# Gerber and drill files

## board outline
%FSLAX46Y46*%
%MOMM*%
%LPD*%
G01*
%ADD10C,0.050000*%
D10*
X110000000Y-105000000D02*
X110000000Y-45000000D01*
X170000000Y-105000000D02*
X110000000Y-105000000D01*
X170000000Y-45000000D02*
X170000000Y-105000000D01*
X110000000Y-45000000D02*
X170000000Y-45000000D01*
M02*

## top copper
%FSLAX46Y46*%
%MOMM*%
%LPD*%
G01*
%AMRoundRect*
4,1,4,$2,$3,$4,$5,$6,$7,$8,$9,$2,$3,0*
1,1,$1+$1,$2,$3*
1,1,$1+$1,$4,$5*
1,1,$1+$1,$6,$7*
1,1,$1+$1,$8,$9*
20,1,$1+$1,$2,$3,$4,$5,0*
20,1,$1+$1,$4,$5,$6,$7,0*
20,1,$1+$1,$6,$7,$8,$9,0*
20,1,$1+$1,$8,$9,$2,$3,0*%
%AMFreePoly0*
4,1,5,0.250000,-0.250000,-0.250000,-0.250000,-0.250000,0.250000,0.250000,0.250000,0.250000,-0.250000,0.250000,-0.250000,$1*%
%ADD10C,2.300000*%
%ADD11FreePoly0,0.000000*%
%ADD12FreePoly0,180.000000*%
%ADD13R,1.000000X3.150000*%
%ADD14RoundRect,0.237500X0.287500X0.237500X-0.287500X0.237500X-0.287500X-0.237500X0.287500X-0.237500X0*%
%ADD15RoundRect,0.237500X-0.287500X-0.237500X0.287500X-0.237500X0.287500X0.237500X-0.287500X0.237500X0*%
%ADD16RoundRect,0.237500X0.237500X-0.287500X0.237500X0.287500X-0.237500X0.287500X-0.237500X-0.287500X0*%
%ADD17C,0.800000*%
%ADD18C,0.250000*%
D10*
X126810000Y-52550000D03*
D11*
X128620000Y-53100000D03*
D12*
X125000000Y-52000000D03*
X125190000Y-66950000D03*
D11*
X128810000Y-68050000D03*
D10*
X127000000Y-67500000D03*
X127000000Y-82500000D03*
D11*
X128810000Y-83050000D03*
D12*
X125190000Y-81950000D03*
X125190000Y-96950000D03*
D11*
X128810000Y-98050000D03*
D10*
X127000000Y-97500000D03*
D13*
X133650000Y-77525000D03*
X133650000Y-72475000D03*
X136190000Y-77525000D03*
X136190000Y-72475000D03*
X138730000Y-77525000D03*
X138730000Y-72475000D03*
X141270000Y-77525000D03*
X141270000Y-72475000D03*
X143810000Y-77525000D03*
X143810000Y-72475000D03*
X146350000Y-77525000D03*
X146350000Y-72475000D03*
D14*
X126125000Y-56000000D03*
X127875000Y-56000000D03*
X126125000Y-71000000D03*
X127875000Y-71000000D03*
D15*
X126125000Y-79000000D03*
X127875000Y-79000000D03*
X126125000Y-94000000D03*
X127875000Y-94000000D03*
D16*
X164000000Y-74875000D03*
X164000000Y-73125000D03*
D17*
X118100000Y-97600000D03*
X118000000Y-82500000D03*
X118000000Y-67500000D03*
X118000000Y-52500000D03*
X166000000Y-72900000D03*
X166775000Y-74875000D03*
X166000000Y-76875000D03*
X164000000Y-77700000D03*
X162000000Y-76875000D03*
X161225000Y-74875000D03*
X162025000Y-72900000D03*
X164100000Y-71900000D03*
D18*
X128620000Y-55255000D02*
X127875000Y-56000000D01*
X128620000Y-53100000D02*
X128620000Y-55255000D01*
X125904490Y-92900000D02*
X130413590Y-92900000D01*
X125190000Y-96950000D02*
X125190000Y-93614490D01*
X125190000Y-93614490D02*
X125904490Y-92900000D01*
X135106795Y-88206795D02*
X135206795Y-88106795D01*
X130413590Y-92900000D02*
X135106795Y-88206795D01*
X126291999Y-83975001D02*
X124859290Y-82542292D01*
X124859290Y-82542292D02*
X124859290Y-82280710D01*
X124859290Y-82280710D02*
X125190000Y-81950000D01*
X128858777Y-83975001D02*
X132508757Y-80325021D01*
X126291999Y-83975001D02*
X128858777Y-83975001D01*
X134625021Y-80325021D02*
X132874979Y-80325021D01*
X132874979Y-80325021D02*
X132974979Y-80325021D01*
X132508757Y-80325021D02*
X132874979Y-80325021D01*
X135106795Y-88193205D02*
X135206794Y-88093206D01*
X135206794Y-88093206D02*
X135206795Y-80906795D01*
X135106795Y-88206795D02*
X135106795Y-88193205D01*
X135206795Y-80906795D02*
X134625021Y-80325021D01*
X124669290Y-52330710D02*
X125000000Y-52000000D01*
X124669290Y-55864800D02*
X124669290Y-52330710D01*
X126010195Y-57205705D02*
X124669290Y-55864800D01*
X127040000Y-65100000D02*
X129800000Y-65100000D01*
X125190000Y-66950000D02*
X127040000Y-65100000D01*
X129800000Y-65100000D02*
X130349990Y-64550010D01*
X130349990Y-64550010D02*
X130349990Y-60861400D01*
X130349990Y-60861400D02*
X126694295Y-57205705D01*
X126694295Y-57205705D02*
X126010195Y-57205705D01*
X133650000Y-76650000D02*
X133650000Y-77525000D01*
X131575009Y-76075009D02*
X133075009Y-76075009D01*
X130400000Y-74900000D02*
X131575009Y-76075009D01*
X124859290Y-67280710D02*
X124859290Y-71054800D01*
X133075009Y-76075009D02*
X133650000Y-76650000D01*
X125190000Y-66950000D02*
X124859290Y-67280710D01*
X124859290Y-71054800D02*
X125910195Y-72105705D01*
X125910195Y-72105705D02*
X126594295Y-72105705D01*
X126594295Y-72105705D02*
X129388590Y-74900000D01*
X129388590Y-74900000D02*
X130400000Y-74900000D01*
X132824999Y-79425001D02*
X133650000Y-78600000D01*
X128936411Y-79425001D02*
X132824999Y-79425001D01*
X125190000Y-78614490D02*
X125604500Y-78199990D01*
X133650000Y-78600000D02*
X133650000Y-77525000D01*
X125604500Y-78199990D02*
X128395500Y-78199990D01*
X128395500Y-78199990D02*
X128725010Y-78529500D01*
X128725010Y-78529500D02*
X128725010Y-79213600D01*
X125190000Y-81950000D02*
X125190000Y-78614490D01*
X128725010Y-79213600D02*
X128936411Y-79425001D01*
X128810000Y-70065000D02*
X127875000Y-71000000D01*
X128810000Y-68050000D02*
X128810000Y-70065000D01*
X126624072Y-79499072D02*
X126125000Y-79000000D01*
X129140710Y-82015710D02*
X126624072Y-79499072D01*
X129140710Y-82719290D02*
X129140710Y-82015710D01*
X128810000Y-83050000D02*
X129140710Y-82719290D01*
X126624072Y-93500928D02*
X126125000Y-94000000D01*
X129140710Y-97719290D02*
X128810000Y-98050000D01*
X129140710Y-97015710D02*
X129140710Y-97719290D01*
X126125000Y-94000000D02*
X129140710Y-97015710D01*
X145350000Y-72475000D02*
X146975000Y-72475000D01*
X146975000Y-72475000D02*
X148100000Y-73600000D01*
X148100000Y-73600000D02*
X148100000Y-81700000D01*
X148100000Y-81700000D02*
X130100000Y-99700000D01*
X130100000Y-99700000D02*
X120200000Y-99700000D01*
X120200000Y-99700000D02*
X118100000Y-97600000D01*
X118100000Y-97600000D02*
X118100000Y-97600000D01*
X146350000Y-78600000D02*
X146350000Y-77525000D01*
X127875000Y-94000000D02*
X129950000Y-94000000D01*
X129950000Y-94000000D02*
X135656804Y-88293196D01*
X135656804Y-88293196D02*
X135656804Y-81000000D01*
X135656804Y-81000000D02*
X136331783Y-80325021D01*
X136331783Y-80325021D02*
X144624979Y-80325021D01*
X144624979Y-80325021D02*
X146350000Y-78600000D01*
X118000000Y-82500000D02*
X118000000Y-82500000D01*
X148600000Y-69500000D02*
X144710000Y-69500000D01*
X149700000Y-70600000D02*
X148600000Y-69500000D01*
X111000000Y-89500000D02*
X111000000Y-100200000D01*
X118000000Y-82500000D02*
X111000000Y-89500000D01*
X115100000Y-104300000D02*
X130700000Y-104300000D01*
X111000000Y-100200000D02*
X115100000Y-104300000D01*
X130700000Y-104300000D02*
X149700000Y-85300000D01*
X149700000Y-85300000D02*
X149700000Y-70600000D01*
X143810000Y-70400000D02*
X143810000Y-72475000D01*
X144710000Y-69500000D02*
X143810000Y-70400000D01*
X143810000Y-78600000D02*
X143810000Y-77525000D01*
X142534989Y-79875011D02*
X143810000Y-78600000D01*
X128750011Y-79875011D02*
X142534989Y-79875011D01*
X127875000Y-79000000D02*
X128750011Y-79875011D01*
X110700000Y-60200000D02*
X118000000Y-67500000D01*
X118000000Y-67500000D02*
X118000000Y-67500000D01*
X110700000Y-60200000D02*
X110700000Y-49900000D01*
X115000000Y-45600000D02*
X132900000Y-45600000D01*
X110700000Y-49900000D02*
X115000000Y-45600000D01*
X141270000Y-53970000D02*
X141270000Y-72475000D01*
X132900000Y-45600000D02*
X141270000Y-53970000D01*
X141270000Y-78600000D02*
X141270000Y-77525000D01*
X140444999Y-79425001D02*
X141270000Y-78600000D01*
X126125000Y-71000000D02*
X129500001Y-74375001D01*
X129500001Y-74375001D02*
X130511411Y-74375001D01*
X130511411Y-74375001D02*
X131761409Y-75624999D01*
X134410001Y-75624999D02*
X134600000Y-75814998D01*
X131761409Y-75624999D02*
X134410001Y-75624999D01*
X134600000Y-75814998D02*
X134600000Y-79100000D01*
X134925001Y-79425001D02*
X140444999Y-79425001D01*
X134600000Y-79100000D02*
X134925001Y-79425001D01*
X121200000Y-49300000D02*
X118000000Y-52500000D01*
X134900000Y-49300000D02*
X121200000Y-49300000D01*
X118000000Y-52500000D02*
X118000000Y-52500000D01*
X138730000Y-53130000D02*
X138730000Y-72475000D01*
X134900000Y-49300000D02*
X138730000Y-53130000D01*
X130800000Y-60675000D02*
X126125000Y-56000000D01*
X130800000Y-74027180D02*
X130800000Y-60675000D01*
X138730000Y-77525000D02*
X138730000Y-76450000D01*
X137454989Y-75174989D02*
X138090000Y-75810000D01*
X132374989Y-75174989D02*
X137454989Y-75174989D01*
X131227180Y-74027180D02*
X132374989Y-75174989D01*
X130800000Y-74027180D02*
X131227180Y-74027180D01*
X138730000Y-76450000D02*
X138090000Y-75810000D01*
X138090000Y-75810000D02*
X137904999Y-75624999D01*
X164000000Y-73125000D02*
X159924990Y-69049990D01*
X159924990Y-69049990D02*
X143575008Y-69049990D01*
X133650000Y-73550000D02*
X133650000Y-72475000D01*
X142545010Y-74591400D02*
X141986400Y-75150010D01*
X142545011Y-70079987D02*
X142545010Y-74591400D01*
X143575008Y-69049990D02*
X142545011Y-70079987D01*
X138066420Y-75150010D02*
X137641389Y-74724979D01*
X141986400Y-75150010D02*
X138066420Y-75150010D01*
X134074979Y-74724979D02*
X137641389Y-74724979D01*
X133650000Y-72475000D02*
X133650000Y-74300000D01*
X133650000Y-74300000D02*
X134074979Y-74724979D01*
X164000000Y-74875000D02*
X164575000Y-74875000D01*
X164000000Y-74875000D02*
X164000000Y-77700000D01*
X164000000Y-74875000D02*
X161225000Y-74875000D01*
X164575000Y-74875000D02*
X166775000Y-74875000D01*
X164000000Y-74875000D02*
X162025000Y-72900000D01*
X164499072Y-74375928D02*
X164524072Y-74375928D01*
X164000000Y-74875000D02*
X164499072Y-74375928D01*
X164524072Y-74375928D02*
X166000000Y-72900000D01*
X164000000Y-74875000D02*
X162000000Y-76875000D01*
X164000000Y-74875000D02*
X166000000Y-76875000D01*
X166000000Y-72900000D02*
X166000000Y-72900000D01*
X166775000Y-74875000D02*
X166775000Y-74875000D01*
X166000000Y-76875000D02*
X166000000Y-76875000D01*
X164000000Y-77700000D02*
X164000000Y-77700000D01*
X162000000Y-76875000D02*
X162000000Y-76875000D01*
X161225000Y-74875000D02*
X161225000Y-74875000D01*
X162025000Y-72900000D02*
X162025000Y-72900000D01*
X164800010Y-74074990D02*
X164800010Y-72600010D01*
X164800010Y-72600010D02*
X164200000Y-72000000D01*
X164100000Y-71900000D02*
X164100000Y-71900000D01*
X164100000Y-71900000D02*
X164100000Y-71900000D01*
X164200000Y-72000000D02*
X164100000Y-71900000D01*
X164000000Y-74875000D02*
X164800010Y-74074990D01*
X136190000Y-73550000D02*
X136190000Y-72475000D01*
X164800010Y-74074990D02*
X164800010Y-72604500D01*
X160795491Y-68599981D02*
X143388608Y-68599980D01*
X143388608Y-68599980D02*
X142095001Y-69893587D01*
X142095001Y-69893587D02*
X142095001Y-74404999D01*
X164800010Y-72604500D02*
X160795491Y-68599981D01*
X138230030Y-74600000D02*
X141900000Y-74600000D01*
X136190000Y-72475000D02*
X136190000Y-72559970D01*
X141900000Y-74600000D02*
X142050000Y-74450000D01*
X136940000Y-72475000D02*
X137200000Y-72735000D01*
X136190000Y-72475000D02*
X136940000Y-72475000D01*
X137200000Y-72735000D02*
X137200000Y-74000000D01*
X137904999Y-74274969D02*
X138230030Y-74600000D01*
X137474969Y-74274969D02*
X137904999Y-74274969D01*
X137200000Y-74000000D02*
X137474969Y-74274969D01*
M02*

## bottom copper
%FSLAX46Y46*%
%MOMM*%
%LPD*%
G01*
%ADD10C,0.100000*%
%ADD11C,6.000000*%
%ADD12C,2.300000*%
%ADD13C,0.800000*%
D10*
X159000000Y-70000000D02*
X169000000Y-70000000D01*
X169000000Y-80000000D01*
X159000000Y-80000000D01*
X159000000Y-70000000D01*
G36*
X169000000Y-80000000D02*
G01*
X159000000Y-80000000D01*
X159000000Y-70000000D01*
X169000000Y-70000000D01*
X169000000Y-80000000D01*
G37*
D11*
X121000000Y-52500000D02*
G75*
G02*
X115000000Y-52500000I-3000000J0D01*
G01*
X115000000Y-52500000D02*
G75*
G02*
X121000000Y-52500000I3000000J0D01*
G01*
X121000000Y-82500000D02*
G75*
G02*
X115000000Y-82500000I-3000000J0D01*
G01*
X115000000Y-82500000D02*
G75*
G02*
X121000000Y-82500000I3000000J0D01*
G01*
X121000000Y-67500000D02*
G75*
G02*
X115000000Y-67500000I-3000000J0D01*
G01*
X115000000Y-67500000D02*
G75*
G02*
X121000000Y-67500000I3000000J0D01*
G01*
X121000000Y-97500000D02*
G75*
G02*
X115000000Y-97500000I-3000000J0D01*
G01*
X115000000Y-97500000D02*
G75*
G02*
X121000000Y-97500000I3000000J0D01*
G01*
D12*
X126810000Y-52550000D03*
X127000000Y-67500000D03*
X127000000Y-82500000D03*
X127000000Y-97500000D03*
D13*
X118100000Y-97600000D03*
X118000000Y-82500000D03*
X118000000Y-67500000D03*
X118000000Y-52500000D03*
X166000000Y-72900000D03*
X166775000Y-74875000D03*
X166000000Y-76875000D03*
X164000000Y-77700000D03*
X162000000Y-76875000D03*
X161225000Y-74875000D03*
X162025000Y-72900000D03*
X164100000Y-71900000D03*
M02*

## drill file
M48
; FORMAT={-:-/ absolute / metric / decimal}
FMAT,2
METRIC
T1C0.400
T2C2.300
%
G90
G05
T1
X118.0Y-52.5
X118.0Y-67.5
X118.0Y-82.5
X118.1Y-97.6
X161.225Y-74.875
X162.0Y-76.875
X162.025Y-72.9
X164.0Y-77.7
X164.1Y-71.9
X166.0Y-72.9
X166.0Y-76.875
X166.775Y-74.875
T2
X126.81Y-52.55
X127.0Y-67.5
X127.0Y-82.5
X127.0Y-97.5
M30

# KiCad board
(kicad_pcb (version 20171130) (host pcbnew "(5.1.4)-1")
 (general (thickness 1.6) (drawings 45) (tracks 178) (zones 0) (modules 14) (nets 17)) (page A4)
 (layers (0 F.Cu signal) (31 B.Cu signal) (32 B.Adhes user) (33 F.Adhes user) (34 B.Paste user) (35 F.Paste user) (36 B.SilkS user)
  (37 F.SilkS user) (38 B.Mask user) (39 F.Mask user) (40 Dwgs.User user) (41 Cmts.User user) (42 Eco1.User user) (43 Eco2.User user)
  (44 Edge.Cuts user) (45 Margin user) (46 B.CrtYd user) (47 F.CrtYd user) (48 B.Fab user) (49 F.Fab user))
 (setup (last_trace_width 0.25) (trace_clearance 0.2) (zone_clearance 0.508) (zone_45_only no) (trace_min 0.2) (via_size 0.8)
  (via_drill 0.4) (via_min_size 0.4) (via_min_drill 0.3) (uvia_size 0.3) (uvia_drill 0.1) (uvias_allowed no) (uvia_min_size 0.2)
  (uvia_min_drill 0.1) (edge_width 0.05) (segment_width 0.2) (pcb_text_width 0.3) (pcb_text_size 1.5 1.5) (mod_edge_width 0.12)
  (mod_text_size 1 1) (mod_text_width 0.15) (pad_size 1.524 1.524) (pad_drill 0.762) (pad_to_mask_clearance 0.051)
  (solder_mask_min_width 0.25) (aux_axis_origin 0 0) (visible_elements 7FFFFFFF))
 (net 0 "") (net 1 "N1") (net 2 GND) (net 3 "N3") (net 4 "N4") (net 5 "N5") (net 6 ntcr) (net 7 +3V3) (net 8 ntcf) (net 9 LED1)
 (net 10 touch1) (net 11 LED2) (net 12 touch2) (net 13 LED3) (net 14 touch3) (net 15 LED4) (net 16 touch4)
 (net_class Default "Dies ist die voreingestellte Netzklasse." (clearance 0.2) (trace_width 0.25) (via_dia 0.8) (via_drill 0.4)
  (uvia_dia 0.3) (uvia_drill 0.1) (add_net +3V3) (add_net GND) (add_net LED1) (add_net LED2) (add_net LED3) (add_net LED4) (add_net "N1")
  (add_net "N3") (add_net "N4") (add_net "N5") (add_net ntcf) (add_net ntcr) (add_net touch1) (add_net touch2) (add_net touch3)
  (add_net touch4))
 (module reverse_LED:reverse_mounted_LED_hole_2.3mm (layer F.Cu) (at 126.81 52.55)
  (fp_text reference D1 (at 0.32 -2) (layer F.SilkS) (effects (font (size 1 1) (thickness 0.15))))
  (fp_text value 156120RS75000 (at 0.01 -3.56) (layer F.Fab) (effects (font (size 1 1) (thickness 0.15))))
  (pad 0 thru_hole circle (at 0 0) (size 2.3 2.3) (drill 2.3) (layers *.Cu *.Mask))
  (pad 2 smd custom (at 1.81 0.55) (size 0.5 0.5) (layers F.Cu F.Paste F.Mask) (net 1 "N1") (zone_connect 0)
   (options (clearance outline) (anchor rect)) (primitives))
  (pad 1 smd custom (at -1.81 -0.55 180) (size 0.5 0.5) (layers F.Cu F.Paste F.Mask) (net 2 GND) (zone_connect 0)
   (options (clearance outline) (anchor rect)) (primitives)))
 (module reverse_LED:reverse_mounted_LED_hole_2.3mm (layer F.Cu) (at 127 67.5)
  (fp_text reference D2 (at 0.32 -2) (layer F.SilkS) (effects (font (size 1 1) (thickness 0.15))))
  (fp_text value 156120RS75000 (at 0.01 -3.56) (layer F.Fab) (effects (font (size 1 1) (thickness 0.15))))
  (pad 1 smd custom (at -1.81 -0.55 180) (size 0.5 0.5) (layers F.Cu F.Paste F.Mask) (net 2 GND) (zone_connect 0)
   (options (clearance outline) (anchor rect)) (primitives))
  (pad 2 smd custom (at 1.81 0.55) (size 0.5 0.5) (layers F.Cu F.Paste F.Mask) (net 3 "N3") (zone_connect 0)
   (options (clearance outline) (anchor rect)) (primitives))
  (pad 0 thru_hole circle (at 0 0) (size 2.3 2.3) (drill 2.3) (layers *.Cu *.Mask)))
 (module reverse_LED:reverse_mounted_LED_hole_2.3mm (layer F.Cu) (at 127 82.5)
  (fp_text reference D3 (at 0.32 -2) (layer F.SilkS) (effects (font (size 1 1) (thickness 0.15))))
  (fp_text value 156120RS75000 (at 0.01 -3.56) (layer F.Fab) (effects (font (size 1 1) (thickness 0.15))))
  (pad 0 thru_hole circle (at 0 0) (size 2.3 2.3) (drill 2.3) (layers *.Cu *.Mask))
  (pad 2 smd custom (at 1.81 0.55) (size 0.5 0.5) (layers F.Cu F.Paste F.Mask) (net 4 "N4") (zone_connect 0)
   (options (clearance outline) (anchor rect)) (primitives))
  (pad 1 smd custom (at -1.81 -0.55 180) (size 0.5 0.5) (layers F.Cu F.Paste F.Mask) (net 2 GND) (zone_connect 0)
   (options (clearance outline) (anchor rect)) (primitives)))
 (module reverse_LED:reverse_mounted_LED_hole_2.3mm (layer F.Cu) (at 127 97.5)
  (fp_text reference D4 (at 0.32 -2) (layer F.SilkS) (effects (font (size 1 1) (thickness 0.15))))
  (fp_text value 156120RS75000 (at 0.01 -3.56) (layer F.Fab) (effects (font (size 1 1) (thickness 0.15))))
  (pad 1 smd custom (at -1.81 -0.55 180) (size 0.5 0.5) (layers F.Cu F.Paste F.Mask) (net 2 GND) (zone_connect 0)
   (options (clearance outline) (anchor rect)) (primitives))
  (pad 2 smd custom (at 1.81 0.55) (size 0.5 0.5) (layers F.Cu F.Paste F.Mask) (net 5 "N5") (zone_connect 0)
   (options (clearance outline) (anchor rect)) (primitives))
  (pad 0 thru_hole circle (at 0 0) (size 2.3 2.3) (drill 2.3) (layers *.Cu *.Mask)))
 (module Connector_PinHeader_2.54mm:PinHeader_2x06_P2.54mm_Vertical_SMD (layer F.Cu) (at 140 75 90)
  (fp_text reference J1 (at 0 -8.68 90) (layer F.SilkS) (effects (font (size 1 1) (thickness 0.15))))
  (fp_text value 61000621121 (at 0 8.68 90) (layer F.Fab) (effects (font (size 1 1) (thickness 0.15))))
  (pad 1 smd rect (at -2.525 -6.35 90) (size 3.15 1) (layers F.Cu F.Paste F.Mask) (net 2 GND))
  (pad 2 smd rect (at 2.525 -6.35 90) (size 3.15 1) (layers F.Cu F.Paste F.Mask) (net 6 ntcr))
  (pad 3 smd rect (at -2.525 -3.81 90) (size 3.15 1) (layers F.Cu F.Paste F.Mask) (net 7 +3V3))
  (pad 4 smd rect (at 2.525 -3.81 90) (size 3.15 1) (layers F.Cu F.Paste F.Mask) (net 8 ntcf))
  (pad 5 smd rect (at -2.525 -1.27 90) (size 3.15 1) (layers F.Cu F.Paste F.Mask) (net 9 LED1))
  (pad 6 smd rect (at 2.525 -1.27 90) (size 3.15 1) (layers F.Cu F.Paste F.Mask) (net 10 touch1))
  (pad 7 smd rect (at -2.525 1.27 90) (size 3.15 1) (layers F.Cu F.Paste F.Mask) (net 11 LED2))
  (pad 8 smd rect (at 2.525 1.27 90) (size 3.15 1) (layers F.Cu F.Paste F.Mask) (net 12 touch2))
  (pad 9 smd rect (at -2.525 3.81 90) (size 3.15 1) (layers F.Cu F.Paste F.Mask) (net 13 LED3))
  (pad 10 smd rect (at 2.525 3.81 90) (size 3.15 1) (layers F.Cu F.Paste F.Mask) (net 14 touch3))
  (pad 11 smd rect (at -2.525 6.35 90) (size 3.15 1) (layers F.Cu F.Paste F.Mask) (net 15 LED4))
  (pad 12 smd rect (at 2.525 6.35 90) (size 3.15 1) (layers F.Cu F.Paste F.Mask) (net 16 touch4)))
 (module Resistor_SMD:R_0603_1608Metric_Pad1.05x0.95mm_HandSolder (layer F.Cu) (at 127 56 180)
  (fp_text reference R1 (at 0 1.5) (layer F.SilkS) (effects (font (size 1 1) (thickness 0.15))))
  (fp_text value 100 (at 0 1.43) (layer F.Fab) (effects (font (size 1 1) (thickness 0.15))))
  (pad 2 smd roundrect (at 0.875 0 180) (size 1.05 0.95) (layers F.Cu F.Paste F.Mask) (roundrect_rratio 0.25) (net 9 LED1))
  (pad 1 smd roundrect (at -0.875 0 180) (size 1.05 0.95) (layers F.Cu F.Paste F.Mask) (roundrect_rratio 0.25) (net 1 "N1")))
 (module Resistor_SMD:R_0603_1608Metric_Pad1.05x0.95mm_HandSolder (layer F.Cu) (at 127 71 180)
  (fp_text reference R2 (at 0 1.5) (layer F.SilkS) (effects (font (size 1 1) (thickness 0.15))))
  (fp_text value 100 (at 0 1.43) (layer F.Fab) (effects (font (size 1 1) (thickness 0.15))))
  (pad 2 smd roundrect (at 0.875 0 180) (size 1.05 0.95) (layers F.Cu F.Paste F.Mask) (roundrect_rratio 0.25) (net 11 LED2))
  (pad 1 smd roundrect (at -0.875 0 180) (size 1.05 0.95) (layers F.Cu F.Paste F.Mask) (roundrect_rratio 0.25) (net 3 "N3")))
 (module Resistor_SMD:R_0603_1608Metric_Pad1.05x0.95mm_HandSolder (layer F.Cu) (at 127 79)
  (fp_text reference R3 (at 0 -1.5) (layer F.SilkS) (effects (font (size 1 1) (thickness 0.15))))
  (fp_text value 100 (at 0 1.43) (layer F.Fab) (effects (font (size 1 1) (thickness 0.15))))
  (pad 1 smd roundrect (at -0.875 0) (size 1.05 0.95) (layers F.Cu F.Paste F.Mask) (roundrect_rratio 0.25) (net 4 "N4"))
  (pad 2 smd roundrect (at 0.875 0) (size 1.05 0.95) (layers F.Cu F.Paste F.Mask) (roundrect_rratio 0.25) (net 13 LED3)))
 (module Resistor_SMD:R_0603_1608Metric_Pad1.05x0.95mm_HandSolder (layer F.Cu) (at 127 94)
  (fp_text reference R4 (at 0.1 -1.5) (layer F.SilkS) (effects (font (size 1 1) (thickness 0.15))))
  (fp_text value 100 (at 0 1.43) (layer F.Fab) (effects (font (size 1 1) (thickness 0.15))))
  (pad 1 smd roundrect (at -0.875 0) (size 1.05 0.95) (layers F.Cu F.Paste F.Mask) (roundrect_rratio 0.25) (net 5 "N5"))
  (pad 2 smd roundrect (at 0.875 0) (size 1.05 0.95) (layers F.Cu F.Paste F.Mask) (roundrect_rratio 0.25) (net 15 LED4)))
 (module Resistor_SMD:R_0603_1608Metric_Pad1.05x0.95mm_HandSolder (layer F.Cu) (at 164 74 90)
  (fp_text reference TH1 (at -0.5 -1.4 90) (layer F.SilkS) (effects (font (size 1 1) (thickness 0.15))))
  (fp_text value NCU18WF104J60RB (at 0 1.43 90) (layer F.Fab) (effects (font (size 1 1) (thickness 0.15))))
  (pad 1 smd roundrect (at -0.875 0 90) (size 1.05 0.95) (layers F.Cu F.Paste F.Mask) (roundrect_rratio 0.25) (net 8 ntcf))
  (pad 2 smd roundrect (at 0.875 0 90) (size 1.05 0.95) (layers F.Cu F.Paste F.Mask) (roundrect_rratio 0.25) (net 6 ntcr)))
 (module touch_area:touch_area (layer F.Cu) (at 118 52.5)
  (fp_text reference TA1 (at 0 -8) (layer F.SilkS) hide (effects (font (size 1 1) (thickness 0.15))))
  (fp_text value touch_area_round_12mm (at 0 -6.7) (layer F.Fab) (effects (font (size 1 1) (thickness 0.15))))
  (fp_circle (center 0 0) (end 3 0) (layer B.Cu) (width 6)))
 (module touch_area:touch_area (layer F.Cu) (at 118 82.5)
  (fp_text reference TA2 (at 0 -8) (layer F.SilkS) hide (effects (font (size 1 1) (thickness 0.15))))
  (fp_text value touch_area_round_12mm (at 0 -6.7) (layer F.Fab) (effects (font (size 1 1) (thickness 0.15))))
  (fp_circle (center 0 0) (end 3 0) (layer B.Cu) (width 6)))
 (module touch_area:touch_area (layer F.Cu) (at 118 67.5)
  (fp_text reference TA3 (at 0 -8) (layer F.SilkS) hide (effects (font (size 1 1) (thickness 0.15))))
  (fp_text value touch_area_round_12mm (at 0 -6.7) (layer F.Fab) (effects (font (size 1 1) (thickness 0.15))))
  (fp_circle (center 0 0) (end 3 0) (layer B.Cu) (width 6)))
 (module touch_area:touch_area (layer F.Cu) (at 118 97.5)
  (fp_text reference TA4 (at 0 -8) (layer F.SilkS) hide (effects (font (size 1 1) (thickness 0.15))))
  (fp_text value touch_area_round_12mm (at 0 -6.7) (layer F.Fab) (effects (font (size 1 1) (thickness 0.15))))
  (fp_circle (center 0 0) (end 3 0) (layer B.Cu) (width 6)))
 (gr_poly (pts (xy 159 70) (xy 169 70) (xy 169 80) (xy 159 80)) (layer B.Cu) (width 0.1))
 (gr_line (start 110 105) (end 110 45) (layer Edge.Cuts) (width 0.05))
 (gr_line (start 170 105) (end 110 105) (layer Edge.Cuts) (width 0.05))
 (gr_line (start 170 45) (end 170 105) (layer Edge.Cuts) (width 0.05))
 (gr_line (start 110 45) (end 170 45) (layer Edge.Cuts) (width 0.05))
 (segment (start 128.62 55.255) (end 127.875 56) (width 0.25) (layer F.Cu) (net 1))
 (segment (start 128.62 53.1) (end 128.62 55.255) (width 0.25) (layer F.Cu) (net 1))
 (segment (start 125.90449 92.9) (end 130.41359 92.9) (width 0.25) (layer F.Cu) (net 2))
 (segment (start 125.19 96.95) (end 125.19 93.61449) (width 0.25) (layer F.Cu) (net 2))
 (segment (start 125.19 93.61449) (end 125.90449 92.9) (width 0.25) (layer F.Cu) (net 2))
 (segment (start 135.106795 88.206795) (end 135.206795 88.106795) (width 0.25) (layer F.Cu) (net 2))
 (segment (start 130.41359 92.9) (end 135.106795 88.206795) (width 0.25) (layer F.Cu) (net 2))
 (segment (start 126.291999 83.975001) (end 124.85929 82.542292) (width 0.25) (layer F.Cu) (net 2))
 (segment (start 124.85929 82.542292) (end 124.85929 82.28071) (width 0.25) (layer F.Cu) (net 2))
 (segment (start 124.85929 82.28071) (end 125.19 81.95) (width 0.25) (layer F.Cu) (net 2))
 (segment (start 128.858777 83.975001) (end 132.508757 80.325021) (width 0.25) (layer F.Cu) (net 2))
 (segment (start 126.291999 83.975001) (end 128.858777 83.975001) (width 0.25) (layer F.Cu) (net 2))
 (segment (start 134.625021 80.325021) (end 132.874979 80.325021) (width 0.25) (layer F.Cu) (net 2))
 (segment (start 132.874979 80.325021) (end 132.974979 80.325021) (width 0.25) (layer F.Cu) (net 2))
 (segment (start 132.508757 80.325021) (end 132.874979 80.325021) (width 0.25) (layer F.Cu) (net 2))
 (segment (start 135.106795 88.193205) (end 135.206794 88.093206) (width 0.25) (layer F.Cu) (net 2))
 (segment (start 135.206794 88.093206) (end 135.206795 80.906795) (width 0.25) (layer F.Cu) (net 2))
 (segment (start 135.106795 88.206795) (end 135.106795 88.193205) (width 0.25) (layer F.Cu) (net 2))
 (segment (start 135.206795 80.906795) (end 134.625021 80.325021) (width 0.25) (layer F.Cu) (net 2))
 (segment (start 124.66929 52.33071) (end 125 52) (width 0.25) (layer F.Cu) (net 2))
 (segment (start 124.66929 55.8648) (end 124.66929 52.33071) (width 0.25) (layer F.Cu) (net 2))
 (segment (start 126.010195 57.205705) (end 124.66929 55.8648) (width 0.25) (layer F.Cu) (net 2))
 (segment (start 127.04 65.1) (end 129.8 65.1) (width 0.25) (layer F.Cu) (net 2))
 (segment (start 125.19 66.95) (end 127.04 65.1) (width 0.25) (layer F.Cu) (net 2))
 (segment (start 129.8 65.1) (end 130.34999 64.55001) (width 0.25) (layer F.Cu) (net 2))
 (segment (start 130.34999 64.55001) (end 130.34999 60.8614) (width 0.25) (layer F.Cu) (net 2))
 (segment (start 130.34999 60.8614) (end 126.694295 57.205705) (width 0.25) (layer F.Cu) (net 2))
 (segment (start 126.694295 57.205705) (end 126.010195 57.205705) (width 0.25) (layer F.Cu) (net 2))
 (segment (start 133.65 76.65) (end 133.65 77.525) (width 0.25) (layer F.Cu) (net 2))
 (segment (start 131.575009 76.075009) (end 133.075009 76.075009) (width 0.25) (layer F.Cu) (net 2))
 (segment (start 130.4 74.9) (end 131.575009 76.075009) (width 0.25) (layer F.Cu) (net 2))
 (segment (start 124.85929 67.28071) (end 124.85929 71.0548) (width 0.25) (layer F.Cu) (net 2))
 (segment (start 133.075009 76.075009) (end 133.65 76.65) (width 0.25) (layer F.Cu) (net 2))
 (segment (start 125.19 66.95) (end 124.85929 67.28071) (width 0.25) (layer F.Cu) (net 2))
 (segment (start 124.85929 71.0548) (end 125.910195 72.105705) (width 0.25) (layer F.Cu) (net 2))
 (segment (start 125.910195 72.105705) (end 126.594295 72.105705) (width 0.25) (layer F.Cu) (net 2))
 (segment (start 126.594295 72.105705) (end 129.38859 74.9) (width 0.25) (layer F.Cu) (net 2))
 (segment (start 129.38859 74.9) (end 130.4 74.9) (width 0.25) (layer F.Cu) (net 2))
 (segment (start 132.824999 79.425001) (end 133.65 78.6) (width 0.25) (layer F.Cu) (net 2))
 (segment (start 128.936411 79.425001) (end 132.824999 79.425001) (width 0.25) (layer F.Cu) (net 2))
 (segment (start 125.19 78.61449) (end 125.6045 78.19999) (width 0.25) (layer F.Cu) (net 2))
 (segment (start 133.65 78.6) (end 133.65 77.525) (width 0.25) (layer F.Cu) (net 2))
 (segment (start 125.6045 78.19999) (end 128.3955 78.19999) (width 0.25) (layer F.Cu) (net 2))
 (segment (start 128.3955 78.19999) (end 128.72501 78.5295) (width 0.25) (layer F.Cu) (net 2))
 (segment (start 128.72501 78.5295) (end 128.72501 79.2136) (width 0.25) (layer F.Cu) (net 2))
 (segment (start 125.19 81.95) (end 125.19 78.61449) (width 0.25) (layer F.Cu) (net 2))
 (segment (start 128.72501 79.2136) (end 128.936411 79.425001) (width 0.25) (layer F.Cu) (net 2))
 (segment (start 128.81 70.065) (end 127.875 71) (width 0.25) (layer F.Cu) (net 3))
 (segment (start 128.81 68.05) (end 128.81 70.065) (width 0.25) (layer F.Cu) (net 3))
 (segment (start 126.624072 79.499072) (end 126.125 79) (width 0.25) (layer F.Cu) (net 4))
 (segment (start 129.14071 82.01571) (end 126.624072 79.499072) (width 0.25) (layer F.Cu) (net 4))
 (segment (start 129.14071 82.71929) (end 129.14071 82.01571) (width 0.25) (layer F.Cu) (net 4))
 (segment (start 128.81 83.05) (end 129.14071 82.71929) (width 0.25) (layer F.Cu) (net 4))
 (segment (start 126.624072 93.500928) (end 126.125 94) (width 0.25) (layer F.Cu) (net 5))
 (segment (start 129.14071 97.71929) (end 128.81 98.05) (width 0.25) (layer F.Cu) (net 5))
 (segment (start 129.14071 97.01571) (end 129.14071 97.71929) (width 0.25) (layer F.Cu) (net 5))
 (segment (start 126.125 94) (end 129.14071 97.01571) (width 0.25) (layer F.Cu) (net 5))
 (segment (start 145.35 72.475) (end 146.975 72.475) (width 0.25) (layer F.Cu) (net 16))
 (segment (start 146.975 72.475) (end 148.1 73.6) (width 0.25) (layer F.Cu) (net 16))
 (segment (start 148.1 73.6) (end 148.1 81.7) (width 0.25) (layer F.Cu) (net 16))
 (segment (start 148.1 81.7) (end 130.1 99.7) (width 0.25) (layer F.Cu) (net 16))
 (segment (start 130.1 99.7) (end 120.2 99.7) (width 0.25) (layer F.Cu) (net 16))
 (segment (start 120.2 99.7) (end 118.1 97.6) (width 0.25) (layer F.Cu) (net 16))
 (segment (start 118.1 97.6) (end 118.1 97.6) (width 0.25) (layer F.Cu) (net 16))
 (via (at 118.1 97.6) (size 0.8) (drill 0.4) (layers F.Cu B.Cu) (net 16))
 (segment (start 146.35 78.6) (end 146.35 77.525) (width 0.25) (layer F.Cu) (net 15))
 (segment (start 127.875 94) (end 129.95 94) (width 0.25) (layer F.Cu) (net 15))
 (segment (start 129.95 94) (end 135.656804 88.293196) (width 0.25) (layer F.Cu) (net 15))
 (segment (start 135.656804 88.293196) (end 135.656804 81) (width 0.25) (layer F.Cu) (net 15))
 (segment (start 135.656804 81) (end 136.331783 80.325021) (width 0.25) (layer F.Cu) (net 15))
 (segment (start 136.331783 80.325021) (end 144.624979 80.325021) (width 0.25) (layer F.Cu) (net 15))
 (segment (start 144.624979 80.325021) (end 146.35 78.6) (width 0.25) (layer F.Cu) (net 15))
 (segment (start 118 82.5) (end 118 82.5) (width 0.25) (layer F.Cu) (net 14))
 (via (at 118 82.5) (size 0.8) (drill 0.4) (layers F.Cu B.Cu) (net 14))
 (segment (start 148.6 69.5) (end 144.71 69.5) (width 0.25) (layer F.Cu) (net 14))
 (segment (start 149.7 70.6) (end 148.6 69.5) (width 0.25) (layer F.Cu) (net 14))
 (segment (start 111 89.5) (end 111 100.2) (width 0.25) (layer F.Cu) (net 14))
 (segment (start 118 82.5) (end 111 89.5) (width 0.25) (layer F.Cu) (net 14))
 (segment (start 115.1 104.3) (end 130.7 104.3) (width 0.25) (layer F.Cu) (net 14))
 (segment (start 111 100.2) (end 115.1 104.3) (width 0.25) (layer F.Cu) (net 14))
 (segment (start 130.7 104.3) (end 149.7 85.3) (width 0.25) (layer F.Cu) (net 14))
 (segment (start 149.7 85.3) (end 149.7 70.6) (width 0.25) (layer F.Cu) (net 14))
 (segment (start 143.81 70.4) (end 143.81 72.475) (width 0.25) (layer F.Cu) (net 14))
 (segment (start 144.71 69.5) (end 143.81 70.4) (width 0.25) (layer F.Cu) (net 14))
 (segment (start 143.81 78.6) (end 143.81 77.525) (width 0.25) (layer F.Cu) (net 13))
 (segment (start 142.534989 79.875011) (end 143.81 78.6) (width 0.25) (layer F.Cu) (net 13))
 (segment (start 128.750011 79.875011) (end 142.534989 79.875011) (width 0.25) (layer F.Cu) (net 13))
 (segment (start 127.875 79) (end 128.750011 79.875011) (width 0.25) (layer F.Cu) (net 13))
 (segment (start 110.7 60.2) (end 118 67.5) (width 0.25) (layer F.Cu) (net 12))
 (segment (start 118 67.5) (end 118 67.5) (width 0.25) (layer F.Cu) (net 12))
 (via (at 118 67.5) (size 0.8) (drill 0.4) (layers F.Cu B.Cu) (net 12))
 (segment (start 110.7 60.2) (end 110.7 49.9) (width 0.25) (layer F.Cu) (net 12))
 (segment (start 115 45.6) (end 132.9 45.6) (width 0.25) (layer F.Cu) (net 12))
 (segment (start 110.7 49.9) (end 115 45.6) (width 0.25) (layer F.Cu) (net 12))
 (segment (start 141.27 53.97) (end 141.27 72.475) (width 0.25) (layer F.Cu) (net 12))
 (segment (start 132.9 45.6) (end 141.27 53.97) (width 0.25) (layer F.Cu) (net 12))
 (segment (start 141.27 78.6) (end 141.27 77.525) (width 0.25) (layer F.Cu) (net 11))
 (segment (start 140.444999 79.425001) (end 141.27 78.6) (width 0.25) (layer F.Cu) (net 11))
 (segment (start 126.125 71) (end 129.500001 74.375001) (width 0.25) (layer F.Cu) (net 11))
 (segment (start 129.500001 74.375001) (end 130.511411 74.375001) (width 0.25) (layer F.Cu) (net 11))
 (segment (start 130.511411 74.375001) (end 131.761409 75.624999) (width 0.25) (layer F.Cu) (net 11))
 (segment (start 134.410001 75.624999) (end 134.6 75.814998) (width 0.25) (layer F.Cu) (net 11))
 (segment (start 131.761409 75.624999) (end 134.410001 75.624999) (width 0.25) (layer F.Cu) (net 11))
 (segment (start 134.6 75.814998) (end 134.6 79.1) (width 0.25) (layer F.Cu) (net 11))
 (segment (start 134.925001 79.425001) (end 140.444999 79.425001) (width 0.25) (layer F.Cu) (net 11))
 (segment (start 134.6 79.1) (end 134.925001 79.425001) (width 0.25) (layer F.Cu) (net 11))
 (segment (start 121.2 49.3) (end 118 52.5) (width 0.25) (layer F.Cu) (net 10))
 (segment (start 134.9 49.3) (end 121.2 49.3) (width 0.25) (layer F.Cu) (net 10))
 (segment (start 118 52.5) (end 118 52.5) (width 0.25) (layer F.Cu) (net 10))
 (via (at 118 52.5) (size 0.8) (drill 0.4) (layers F.Cu B.Cu) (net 10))
 (segment (start 138.73 53.13) (end 138.73 72.475) (width 0.25) (layer F.Cu) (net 10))
 (segment (start 134.9 49.3) (end 138.73 53.13) (width 0.25) (layer F.Cu) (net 10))
 (segment (start 130.8 60.675) (end 126.125 56) (width 0.25) (layer F.Cu) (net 9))
 (segment (start 130.8 74.02718) (end 130.8 60.675) (width 0.25) (layer F.Cu) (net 9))
 (segment (start 138.73 77.525) (end 138.73 76.45) (width 0.25) (layer F.Cu) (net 9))
 (segment (start 137.454989 75.174989) (end 138.09 75.81) (width 0.25) (layer F.Cu) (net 9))
 (segment (start 132.374989 75.174989) (end 137.454989 75.174989) (width 0.25) (layer F.Cu) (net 9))
 (segment (start 131.22718 74.02718) (end 132.374989 75.174989) (width 0.25) (layer F.Cu) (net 9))
 (segment (start 130.8 74.02718) (end 131.22718 74.02718) (width 0.25) (layer F.Cu) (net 9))
 (segment (start 138.73 76.45) (end 138.09 75.81) (width 0.25) (layer F.Cu) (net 9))
 (segment (start 138.09 75.81) (end 137.904999 75.624999) (width 0.25) (layer F.Cu) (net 9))
 (segment (start 164 73.125) (end 159.92499 69.04999) (width 0.25) (layer F.Cu) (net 6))
 (segment (start 159.92499 69.04999) (end 143.575008 69.04999) (width 0.25) (layer F.Cu) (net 6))
 (segment (start 133.65 73.55) (end 133.65 72.475) (width 0.25) (layer F.Cu) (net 6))
 (segment (start 142.54501 74.5914) (end 141.9864 75.15001) (width 0.25) (layer F.Cu) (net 6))
 (segment (start 142.545011 70.079987) (end 142.54501 74.5914) (width 0.25) (layer F.Cu) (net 6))
 (segment (start 143.575008 69.04999) (end 142.545011 70.079987) (width 0.25) (layer F.Cu) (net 6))
 (segment (start 138.06642 75.15001) (end 137.641389 74.724979) (width 0.25) (layer F.Cu) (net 6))
 (segment (start 141.9864 75.15001) (end 138.06642 75.15001) (width 0.25) (layer F.Cu) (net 6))
 (segment (start 134.074979 74.724979) (end 137.641389 74.724979) (width 0.25) (layer F.Cu) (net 6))
 (segment (start 133.65 72.475) (end 133.65 74.3) (width 0.25) (layer F.Cu) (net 6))
 (segment (start 133.65 74.3) (end 134.074979 74.724979) (width 0.25) (layer F.Cu) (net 6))
 (segment (start 164 74.875) (end 164.575 74.875) (width 0.25) (layer F.Cu) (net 8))
 (segment (start 164 74.875) (end 164 77.7) (width 0.25) (layer F.Cu) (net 8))
 (segment (start 164 74.875) (end 161.225 74.875) (width 0.25) (layer F.Cu) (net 8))
 (segment (start 164.575 74.875) (end 166.775 74.875) (width 0.25) (layer F.Cu) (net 8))
 (segment (start 164 74.875) (end 162.025 72.9) (width 0.25) (layer F.Cu) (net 8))
 (segment (start 164.499072 74.375928) (end 164.524072 74.375928) (width 0.25) (layer F.Cu) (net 8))
 (segment (start 164 74.875) (end 164.499072 74.375928) (width 0.25) (layer F.Cu) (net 8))
 (segment (start 164.524072 74.375928) (end 166 72.9) (width 0.25) (layer F.Cu) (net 8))
 (segment (start 164 74.875) (end 162 76.875) (width 0.25) (layer F.Cu) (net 8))
 (segment (start 164 74.875) (end 166 76.875) (width 0.25) (layer F.Cu) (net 8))
 (segment (start 166 72.9) (end 166 72.9) (width 0.25) (layer F.Cu) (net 8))
 (via (at 166 72.9) (size 0.8) (drill 0.4) (layers F.Cu B.Cu) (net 8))
 (segment (start 166.775 74.875) (end 166.775 74.875) (width 0.25) (layer F.Cu) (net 8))
 (via (at 166.775 74.875) (size 0.8) (drill 0.4) (layers F.Cu B.Cu) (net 8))
 (segment (start 166 76.875) (end 166 76.875) (width 0.25) (layer F.Cu) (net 8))
 (via (at 166 76.875) (size 0.8) (drill 0.4) (layers F.Cu B.Cu) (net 8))
 (segment (start 164 77.7) (end 164 77.7) (width 0.25) (layer F.Cu) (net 8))
 (via (at 164 77.7) (size 0.8) (drill 0.4) (layers F.Cu B.Cu) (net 8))
 (segment (start 162 76.875) (end 162 76.875) (width 0.25) (layer F.Cu) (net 8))
 (via (at 162 76.875) (size 0.8) (drill 0.4) (layers F.Cu B.Cu) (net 8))
 (segment (start 161.225 74.875) (end 161.225 74.875) (width 0.25) (layer F.Cu) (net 8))
 (via (at 161.225 74.875) (size 0.8) (drill 0.4) (layers F.Cu B.Cu) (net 8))
 (segment (start 162.025 72.9) (end 162.025 72.9) (width 0.25) (layer F.Cu) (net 8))
 (via (at 162.025 72.9) (size 0.8) (drill 0.4) (layers F.Cu B.Cu) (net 8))
 (segment (start 164.80001 74.07499) (end 164.80001 72.60001) (width 0.25) (layer F.Cu) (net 8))
 (segment (start 164.80001 72.60001) (end 164.2 72) (width 0.25) (layer F.Cu) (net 8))
 (segment (start 164.1 71.9) (end 164.1 71.9) (width 0.25) (layer F.Cu) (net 8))
 (segment (start 164.1 71.9) (end 164.1 71.9) (width 0.25) (layer F.Cu) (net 8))
 (segment (start 164.2 72) (end 164.1 71.9) (width 0.25) (layer F.Cu) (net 8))
 (via (at 164.1 71.9) (size 0.8) (drill 0.4) (layers F.Cu B.Cu) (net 8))
 (segment (start 164 74.875) (end 164.80001 74.07499) (width 0.25) (layer F.Cu) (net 8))
 (segment (start 136.19 73.55) (end 136.19 72.475) (width 0.25) (layer F.Cu) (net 8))
 (segment (start 164.80001 74.07499) (end 164.80001 72.6045) (width 0.25) (layer F.Cu) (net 8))
 (segment (start 160.795491 68.599981) (end 143.388608 68.59998) (width 0.25) (layer F.Cu) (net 8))
 (segment (start 143.388608 68.59998) (end 142.095001 69.893587) (width 0.25) (layer F.Cu) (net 8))
 (segment (start 142.095001 69.893587) (end 142.095001 74.404999) (width 0.25) (layer F.Cu) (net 8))
 (segment (start 164.80001 72.6045) (end 160.795491 68.599981) (width 0.25) (layer F.Cu) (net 8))
 (segment (start 138.23003 74.6) (end 141.9 74.6) (width 0.25) (layer F.Cu) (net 8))
 (segment (start 136.19 72.475) (end 136.19 72.55997) (width 0.25) (layer F.Cu) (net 8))
 (segment (start 141.9 74.6) (end 142.05 74.45) (width 0.25) (layer F.Cu) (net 8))
 (segment (start 136.94 72.475) (end 137.2 72.735) (width 0.25) (layer F.Cu) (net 8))
 (segment (start 136.19 72.475) (end 136.94 72.475) (width 0.25) (layer F.Cu) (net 8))
 (segment (start 137.2 72.735) (end 137.2 74) (width 0.25) (layer F.Cu) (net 8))
 (segment (start 137.904999 74.274969) (end 138.23003 74.6) (width 0.25) (layer F.Cu) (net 8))
 (segment (start 137.474969 74.274969) (end 137.904999 74.274969) (width 0.25) (layer F.Cu) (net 8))
 (segment (start 137.2 74) (end 137.474969 74.274969) (width 0.25) (layer F.Cu) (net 8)))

